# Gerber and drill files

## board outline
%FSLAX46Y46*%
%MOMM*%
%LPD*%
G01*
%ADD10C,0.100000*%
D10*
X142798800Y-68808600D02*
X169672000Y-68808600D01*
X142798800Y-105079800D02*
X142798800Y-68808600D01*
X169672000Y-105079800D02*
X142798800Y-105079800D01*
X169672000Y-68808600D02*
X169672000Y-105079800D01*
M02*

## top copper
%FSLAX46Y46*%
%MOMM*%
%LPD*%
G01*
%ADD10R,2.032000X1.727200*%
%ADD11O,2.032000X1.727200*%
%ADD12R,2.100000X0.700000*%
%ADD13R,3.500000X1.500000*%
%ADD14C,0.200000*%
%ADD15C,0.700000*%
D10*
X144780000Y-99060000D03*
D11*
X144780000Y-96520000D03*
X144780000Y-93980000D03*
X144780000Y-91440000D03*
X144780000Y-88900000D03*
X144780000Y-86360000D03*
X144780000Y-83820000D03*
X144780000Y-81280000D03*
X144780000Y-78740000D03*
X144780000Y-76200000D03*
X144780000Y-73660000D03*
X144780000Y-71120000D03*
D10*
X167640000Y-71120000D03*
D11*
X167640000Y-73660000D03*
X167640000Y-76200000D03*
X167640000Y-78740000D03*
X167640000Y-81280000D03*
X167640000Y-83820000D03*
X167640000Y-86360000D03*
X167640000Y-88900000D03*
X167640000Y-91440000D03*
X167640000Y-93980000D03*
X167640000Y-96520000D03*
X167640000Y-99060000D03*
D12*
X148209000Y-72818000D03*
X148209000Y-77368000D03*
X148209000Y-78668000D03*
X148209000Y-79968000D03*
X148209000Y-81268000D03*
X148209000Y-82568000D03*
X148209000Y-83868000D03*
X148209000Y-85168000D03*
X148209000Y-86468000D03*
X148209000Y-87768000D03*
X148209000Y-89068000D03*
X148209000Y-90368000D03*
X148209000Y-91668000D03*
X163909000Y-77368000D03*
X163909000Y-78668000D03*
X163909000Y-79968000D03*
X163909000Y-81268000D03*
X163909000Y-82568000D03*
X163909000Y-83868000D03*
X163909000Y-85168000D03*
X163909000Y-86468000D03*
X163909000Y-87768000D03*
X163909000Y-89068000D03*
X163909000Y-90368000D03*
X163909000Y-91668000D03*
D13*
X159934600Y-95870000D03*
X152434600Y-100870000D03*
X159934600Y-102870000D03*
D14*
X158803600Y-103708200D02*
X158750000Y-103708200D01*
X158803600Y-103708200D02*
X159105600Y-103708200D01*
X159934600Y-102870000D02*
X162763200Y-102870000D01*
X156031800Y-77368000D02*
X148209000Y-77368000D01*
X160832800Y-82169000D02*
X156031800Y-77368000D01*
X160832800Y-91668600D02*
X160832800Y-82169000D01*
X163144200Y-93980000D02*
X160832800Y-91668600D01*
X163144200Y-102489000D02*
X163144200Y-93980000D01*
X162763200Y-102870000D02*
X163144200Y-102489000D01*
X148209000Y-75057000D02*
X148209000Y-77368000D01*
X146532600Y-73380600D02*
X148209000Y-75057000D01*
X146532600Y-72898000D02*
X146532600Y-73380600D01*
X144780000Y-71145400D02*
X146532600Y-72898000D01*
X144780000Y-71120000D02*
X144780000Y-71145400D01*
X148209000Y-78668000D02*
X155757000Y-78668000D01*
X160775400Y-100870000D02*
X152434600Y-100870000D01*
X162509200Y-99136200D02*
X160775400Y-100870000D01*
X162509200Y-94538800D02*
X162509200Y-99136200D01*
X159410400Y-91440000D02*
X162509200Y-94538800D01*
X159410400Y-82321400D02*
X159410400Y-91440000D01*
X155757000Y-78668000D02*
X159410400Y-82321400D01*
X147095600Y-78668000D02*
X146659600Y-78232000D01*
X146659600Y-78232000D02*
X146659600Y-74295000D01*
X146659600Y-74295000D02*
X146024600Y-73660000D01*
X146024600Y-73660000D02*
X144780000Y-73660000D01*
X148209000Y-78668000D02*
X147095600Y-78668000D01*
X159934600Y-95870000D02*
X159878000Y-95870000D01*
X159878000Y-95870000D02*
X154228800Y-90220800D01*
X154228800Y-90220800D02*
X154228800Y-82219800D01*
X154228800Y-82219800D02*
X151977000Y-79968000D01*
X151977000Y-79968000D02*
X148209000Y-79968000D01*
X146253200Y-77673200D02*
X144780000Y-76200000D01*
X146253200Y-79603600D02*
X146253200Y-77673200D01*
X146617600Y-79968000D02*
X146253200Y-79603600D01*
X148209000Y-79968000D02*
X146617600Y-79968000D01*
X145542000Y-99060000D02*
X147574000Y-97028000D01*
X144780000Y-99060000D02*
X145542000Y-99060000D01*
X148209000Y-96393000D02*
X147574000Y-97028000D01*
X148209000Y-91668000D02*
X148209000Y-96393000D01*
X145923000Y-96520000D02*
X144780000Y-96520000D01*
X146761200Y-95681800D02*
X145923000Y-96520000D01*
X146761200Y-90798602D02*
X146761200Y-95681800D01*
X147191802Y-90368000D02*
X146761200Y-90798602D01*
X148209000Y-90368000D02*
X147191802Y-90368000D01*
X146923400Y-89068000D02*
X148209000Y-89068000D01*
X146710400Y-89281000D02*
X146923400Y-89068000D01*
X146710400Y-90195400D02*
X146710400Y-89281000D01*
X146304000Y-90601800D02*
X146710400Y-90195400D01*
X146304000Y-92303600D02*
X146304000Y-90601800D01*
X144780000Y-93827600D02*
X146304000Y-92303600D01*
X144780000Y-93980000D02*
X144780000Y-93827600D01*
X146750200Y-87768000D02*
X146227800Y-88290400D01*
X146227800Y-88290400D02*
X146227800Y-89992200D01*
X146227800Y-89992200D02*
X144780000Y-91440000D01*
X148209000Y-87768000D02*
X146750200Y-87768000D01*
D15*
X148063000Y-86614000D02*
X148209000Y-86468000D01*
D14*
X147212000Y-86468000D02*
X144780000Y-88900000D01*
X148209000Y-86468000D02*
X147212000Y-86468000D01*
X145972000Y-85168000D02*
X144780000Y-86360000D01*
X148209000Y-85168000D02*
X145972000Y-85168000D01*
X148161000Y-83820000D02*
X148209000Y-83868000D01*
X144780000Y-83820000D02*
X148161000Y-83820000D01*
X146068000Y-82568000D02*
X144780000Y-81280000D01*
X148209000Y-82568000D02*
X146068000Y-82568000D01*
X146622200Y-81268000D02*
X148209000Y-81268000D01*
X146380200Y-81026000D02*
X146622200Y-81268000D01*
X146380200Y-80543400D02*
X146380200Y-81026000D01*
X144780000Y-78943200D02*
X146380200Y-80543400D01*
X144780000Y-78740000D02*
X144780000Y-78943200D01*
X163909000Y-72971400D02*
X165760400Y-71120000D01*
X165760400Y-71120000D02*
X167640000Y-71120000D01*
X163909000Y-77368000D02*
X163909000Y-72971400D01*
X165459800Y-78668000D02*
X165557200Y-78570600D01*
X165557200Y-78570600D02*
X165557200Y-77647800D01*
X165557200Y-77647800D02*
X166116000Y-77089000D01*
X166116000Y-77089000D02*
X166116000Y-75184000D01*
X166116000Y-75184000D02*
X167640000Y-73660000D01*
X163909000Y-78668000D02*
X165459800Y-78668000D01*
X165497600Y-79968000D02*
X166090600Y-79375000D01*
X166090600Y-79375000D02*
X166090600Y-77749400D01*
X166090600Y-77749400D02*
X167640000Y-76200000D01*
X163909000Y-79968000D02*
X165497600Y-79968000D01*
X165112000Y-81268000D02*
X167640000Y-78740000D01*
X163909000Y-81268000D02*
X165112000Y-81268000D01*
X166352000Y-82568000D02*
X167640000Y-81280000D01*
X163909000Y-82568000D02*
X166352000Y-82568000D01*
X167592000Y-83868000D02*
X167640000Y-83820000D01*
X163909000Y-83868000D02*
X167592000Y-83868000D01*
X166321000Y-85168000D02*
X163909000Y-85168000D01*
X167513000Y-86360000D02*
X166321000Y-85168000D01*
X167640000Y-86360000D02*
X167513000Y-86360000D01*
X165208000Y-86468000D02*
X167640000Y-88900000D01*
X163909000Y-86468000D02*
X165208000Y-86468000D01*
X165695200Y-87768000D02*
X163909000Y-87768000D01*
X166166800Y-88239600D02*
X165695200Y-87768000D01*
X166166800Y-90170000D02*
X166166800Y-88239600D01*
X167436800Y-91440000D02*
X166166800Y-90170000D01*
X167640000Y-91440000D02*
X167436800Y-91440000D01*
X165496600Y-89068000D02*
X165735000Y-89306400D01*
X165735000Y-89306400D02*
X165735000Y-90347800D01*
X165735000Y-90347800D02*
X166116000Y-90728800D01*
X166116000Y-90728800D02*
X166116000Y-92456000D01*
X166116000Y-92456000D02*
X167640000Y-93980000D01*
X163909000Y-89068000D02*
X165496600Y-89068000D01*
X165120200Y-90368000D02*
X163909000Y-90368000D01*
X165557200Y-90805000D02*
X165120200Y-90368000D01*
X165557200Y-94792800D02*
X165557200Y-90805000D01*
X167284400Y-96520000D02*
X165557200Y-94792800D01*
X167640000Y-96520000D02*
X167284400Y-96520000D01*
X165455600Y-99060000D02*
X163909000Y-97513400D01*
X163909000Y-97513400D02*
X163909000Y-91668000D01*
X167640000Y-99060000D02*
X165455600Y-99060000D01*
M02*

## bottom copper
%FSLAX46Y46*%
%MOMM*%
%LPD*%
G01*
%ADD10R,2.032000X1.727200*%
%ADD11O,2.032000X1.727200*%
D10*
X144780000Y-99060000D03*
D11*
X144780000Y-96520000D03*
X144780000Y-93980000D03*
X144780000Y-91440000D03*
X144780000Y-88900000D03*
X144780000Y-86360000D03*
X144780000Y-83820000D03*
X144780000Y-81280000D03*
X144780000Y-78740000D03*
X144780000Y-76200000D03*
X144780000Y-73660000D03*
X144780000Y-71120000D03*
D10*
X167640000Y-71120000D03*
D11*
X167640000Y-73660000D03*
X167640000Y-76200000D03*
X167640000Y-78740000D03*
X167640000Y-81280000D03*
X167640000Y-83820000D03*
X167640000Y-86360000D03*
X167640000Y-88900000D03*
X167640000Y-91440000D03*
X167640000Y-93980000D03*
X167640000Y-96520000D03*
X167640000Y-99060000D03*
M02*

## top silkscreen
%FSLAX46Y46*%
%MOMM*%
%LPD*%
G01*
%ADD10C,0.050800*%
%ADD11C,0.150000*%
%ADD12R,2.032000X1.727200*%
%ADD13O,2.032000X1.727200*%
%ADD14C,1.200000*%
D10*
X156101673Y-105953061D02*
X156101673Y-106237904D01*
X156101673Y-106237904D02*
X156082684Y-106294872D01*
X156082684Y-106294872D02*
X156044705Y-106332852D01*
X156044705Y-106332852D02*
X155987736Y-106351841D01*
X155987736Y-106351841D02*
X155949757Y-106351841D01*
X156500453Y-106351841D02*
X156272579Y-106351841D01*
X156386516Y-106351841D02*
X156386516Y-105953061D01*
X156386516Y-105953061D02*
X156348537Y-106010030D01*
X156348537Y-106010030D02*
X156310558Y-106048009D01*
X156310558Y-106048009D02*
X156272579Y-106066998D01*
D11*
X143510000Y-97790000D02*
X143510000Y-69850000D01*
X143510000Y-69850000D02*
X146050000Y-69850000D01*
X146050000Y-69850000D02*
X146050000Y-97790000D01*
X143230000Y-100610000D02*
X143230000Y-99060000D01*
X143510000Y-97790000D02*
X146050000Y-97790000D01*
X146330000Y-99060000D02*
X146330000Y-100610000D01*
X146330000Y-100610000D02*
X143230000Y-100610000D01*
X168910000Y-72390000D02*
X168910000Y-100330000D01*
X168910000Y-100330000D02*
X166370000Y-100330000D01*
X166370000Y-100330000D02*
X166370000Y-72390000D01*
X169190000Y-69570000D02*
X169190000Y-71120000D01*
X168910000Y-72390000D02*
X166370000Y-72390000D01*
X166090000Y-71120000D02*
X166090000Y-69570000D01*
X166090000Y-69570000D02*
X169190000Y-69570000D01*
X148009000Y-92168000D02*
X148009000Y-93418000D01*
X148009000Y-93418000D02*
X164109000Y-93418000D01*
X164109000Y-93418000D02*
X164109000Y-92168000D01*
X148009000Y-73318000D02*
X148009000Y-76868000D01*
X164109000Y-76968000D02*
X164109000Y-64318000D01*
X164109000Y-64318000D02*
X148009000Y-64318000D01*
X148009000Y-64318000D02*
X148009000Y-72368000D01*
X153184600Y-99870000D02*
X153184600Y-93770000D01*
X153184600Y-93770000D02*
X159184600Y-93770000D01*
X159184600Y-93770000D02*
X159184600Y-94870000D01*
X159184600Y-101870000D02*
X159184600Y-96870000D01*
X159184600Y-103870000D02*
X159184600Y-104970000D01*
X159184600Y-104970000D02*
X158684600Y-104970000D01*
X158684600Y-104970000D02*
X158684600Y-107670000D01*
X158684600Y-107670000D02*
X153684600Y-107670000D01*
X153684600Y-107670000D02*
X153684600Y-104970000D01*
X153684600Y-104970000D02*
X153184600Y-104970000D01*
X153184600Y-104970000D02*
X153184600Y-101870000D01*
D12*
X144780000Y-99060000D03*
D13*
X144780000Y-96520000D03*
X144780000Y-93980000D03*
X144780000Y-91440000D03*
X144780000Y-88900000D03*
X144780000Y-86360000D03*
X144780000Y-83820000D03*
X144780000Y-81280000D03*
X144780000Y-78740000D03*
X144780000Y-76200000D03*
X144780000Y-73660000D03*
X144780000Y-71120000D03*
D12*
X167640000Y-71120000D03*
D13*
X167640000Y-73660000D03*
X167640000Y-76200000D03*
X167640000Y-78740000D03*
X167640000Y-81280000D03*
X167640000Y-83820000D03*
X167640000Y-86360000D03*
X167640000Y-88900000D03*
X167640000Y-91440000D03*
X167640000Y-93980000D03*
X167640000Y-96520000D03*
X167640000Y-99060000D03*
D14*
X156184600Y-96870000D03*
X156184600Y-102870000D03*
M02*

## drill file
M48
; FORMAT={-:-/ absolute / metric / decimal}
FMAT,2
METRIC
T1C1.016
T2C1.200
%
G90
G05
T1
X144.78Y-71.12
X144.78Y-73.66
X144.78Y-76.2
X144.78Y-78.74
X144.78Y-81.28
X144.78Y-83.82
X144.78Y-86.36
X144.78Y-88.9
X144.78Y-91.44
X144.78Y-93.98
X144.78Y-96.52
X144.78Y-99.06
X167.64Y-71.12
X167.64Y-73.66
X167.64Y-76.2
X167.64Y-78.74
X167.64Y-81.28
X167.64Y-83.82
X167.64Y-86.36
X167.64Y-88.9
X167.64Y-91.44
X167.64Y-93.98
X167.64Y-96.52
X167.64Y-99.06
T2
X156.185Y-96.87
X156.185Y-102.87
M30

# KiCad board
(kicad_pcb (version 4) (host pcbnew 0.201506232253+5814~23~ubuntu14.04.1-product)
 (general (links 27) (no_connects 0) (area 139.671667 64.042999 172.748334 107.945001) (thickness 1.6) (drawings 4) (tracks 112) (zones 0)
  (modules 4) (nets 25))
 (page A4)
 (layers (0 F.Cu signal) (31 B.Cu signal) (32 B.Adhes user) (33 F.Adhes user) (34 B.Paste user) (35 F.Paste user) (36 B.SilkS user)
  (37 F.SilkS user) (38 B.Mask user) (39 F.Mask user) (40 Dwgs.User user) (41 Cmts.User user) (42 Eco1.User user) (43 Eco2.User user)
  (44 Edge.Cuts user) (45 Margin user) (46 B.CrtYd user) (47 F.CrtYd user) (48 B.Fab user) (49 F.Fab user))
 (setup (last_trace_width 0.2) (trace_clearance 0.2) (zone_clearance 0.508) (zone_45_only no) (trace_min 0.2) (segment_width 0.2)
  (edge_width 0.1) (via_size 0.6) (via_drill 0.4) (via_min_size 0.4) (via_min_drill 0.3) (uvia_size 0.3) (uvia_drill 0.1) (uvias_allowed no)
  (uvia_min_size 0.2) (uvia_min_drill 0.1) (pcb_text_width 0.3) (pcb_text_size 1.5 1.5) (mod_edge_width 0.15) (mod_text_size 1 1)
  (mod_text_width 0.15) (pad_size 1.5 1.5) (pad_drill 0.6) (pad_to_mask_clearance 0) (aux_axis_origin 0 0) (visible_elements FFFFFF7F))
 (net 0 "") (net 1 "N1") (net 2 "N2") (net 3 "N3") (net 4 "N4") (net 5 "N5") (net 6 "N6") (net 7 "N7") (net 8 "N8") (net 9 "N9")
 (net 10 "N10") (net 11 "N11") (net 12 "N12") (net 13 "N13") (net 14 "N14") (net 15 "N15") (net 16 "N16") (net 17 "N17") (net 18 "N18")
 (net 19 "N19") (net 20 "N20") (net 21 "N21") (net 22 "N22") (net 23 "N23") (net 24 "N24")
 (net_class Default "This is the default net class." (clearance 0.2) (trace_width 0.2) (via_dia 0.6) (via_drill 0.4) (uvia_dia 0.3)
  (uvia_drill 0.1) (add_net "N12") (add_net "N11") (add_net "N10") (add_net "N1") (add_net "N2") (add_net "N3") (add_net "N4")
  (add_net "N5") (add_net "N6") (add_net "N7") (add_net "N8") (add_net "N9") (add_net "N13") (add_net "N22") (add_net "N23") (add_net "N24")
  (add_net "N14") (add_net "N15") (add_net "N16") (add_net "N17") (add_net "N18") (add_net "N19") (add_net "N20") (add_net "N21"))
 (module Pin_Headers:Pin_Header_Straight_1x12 (layer F.Cu) (at 144.78 99.06 180)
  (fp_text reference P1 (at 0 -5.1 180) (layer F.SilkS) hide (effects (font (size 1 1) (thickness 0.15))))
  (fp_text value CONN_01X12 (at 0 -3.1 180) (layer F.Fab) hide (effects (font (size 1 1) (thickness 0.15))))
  (fp_line (start 1.27 1.27) (end 1.27 29.21) (layer F.SilkS) (width 0.15))
  (fp_line (start 1.27 29.21) (end -1.27 29.21) (layer F.SilkS) (width 0.15))
  (fp_line (start -1.27 29.21) (end -1.27 1.27) (layer F.SilkS) (width 0.15))
  (fp_line (start 1.55 -1.55) (end 1.55 0) (layer F.SilkS) (width 0.15))
  (fp_line (start 1.27 1.27) (end -1.27 1.27) (layer F.SilkS) (width 0.15))
  (fp_line (start -1.55 0) (end -1.55 -1.55) (layer F.SilkS) (width 0.15))
  (fp_line (start -1.55 -1.55) (end 1.55 -1.55) (layer F.SilkS) (width 0.15))
  (pad 1 thru_hole rect (at 0 0 180) (size 2.032 1.7272) (drill 1.016) (layers *.Cu *.Mask F.SilkS) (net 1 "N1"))
  (pad 2 thru_hole oval (at 0 2.54 180) (size 2.032 1.7272) (drill 1.016) (layers *.Cu *.Mask F.SilkS) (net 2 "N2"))
  (pad 3 thru_hole oval (at 0 5.08 180) (size 2.032 1.7272) (drill 1.016) (layers *.Cu *.Mask F.SilkS) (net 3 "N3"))
  (pad 4 thru_hole oval (at 0 7.62 180) (size 2.032 1.7272) (drill 1.016) (layers *.Cu *.Mask F.SilkS) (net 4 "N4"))
  (pad 5 thru_hole oval (at 0 10.16 180) (size 2.032 1.7272) (drill 1.016) (layers *.Cu *.Mask F.SilkS) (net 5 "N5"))
  (pad 6 thru_hole oval (at 0 12.7 180) (size 2.032 1.7272) (drill 1.016) (layers *.Cu *.Mask F.SilkS) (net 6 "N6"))
  (pad 7 thru_hole oval (at 0 15.24 180) (size 2.032 1.7272) (drill 1.016) (layers *.Cu *.Mask F.SilkS) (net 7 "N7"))
  (pad 8 thru_hole oval (at 0 17.78 180) (size 2.032 1.7272) (drill 1.016) (layers *.Cu *.Mask F.SilkS) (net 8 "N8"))
  (pad 9 thru_hole oval (at 0 20.32 180) (size 2.032 1.7272) (drill 1.016) (layers *.Cu *.Mask F.SilkS) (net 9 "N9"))
  (pad 10 thru_hole oval (at 0 22.86 180) (size 2.032 1.7272) (drill 1.016) (layers *.Cu *.Mask F.SilkS) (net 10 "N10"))
  (pad 11 thru_hole oval (at 0 25.4 180) (size 2.032 1.7272) (drill 1.016) (layers *.Cu *.Mask F.SilkS) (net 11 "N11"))
  (pad 12 thru_hole oval (at 0 27.94 180) (size 2.032 1.7272) (drill 1.016) (layers *.Cu *.Mask F.SilkS) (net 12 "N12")))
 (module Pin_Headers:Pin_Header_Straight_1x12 (layer F.Cu) (at 167.64 71.12)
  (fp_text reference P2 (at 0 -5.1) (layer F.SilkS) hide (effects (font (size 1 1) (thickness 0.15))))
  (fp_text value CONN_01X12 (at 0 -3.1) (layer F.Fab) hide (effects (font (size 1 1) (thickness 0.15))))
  (fp_line (start 1.27 1.27) (end 1.27 29.21) (layer F.SilkS) (width 0.15))
  (fp_line (start 1.27 29.21) (end -1.27 29.21) (layer F.SilkS) (width 0.15))
  (fp_line (start -1.27 29.21) (end -1.27 1.27) (layer F.SilkS) (width 0.15))
  (fp_line (start 1.55 -1.55) (end 1.55 0) (layer F.SilkS) (width 0.15))
  (fp_line (start 1.27 1.27) (end -1.27 1.27) (layer F.SilkS) (width 0.15))
  (fp_line (start -1.55 0) (end -1.55 -1.55) (layer F.SilkS) (width 0.15))
  (fp_line (start -1.55 -1.55) (end 1.55 -1.55) (layer F.SilkS) (width 0.15))
  (pad 1 thru_hole rect (at 0 0) (size 2.032 1.7272) (drill 1.016) (layers *.Cu *.Mask F.SilkS) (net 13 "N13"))
  (pad 2 thru_hole oval (at 0 2.54) (size 2.032 1.7272) (drill 1.016) (layers *.Cu *.Mask F.SilkS) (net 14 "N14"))
  (pad 3 thru_hole oval (at 0 5.08) (size 2.032 1.7272) (drill 1.016) (layers *.Cu *.Mask F.SilkS) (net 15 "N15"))
  (pad 4 thru_hole oval (at 0 7.62) (size 2.032 1.7272) (drill 1.016) (layers *.Cu *.Mask F.SilkS) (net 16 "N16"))
  (pad 5 thru_hole oval (at 0 10.16) (size 2.032 1.7272) (drill 1.016) (layers *.Cu *.Mask F.SilkS) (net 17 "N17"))
  (pad 6 thru_hole oval (at 0 12.7) (size 2.032 1.7272) (drill 1.016) (layers *.Cu *.Mask F.SilkS) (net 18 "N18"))
  (pad 7 thru_hole oval (at 0 15.24) (size 2.032 1.7272) (drill 1.016) (layers *.Cu *.Mask F.SilkS) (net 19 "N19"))
  (pad 8 thru_hole oval (at 0 17.78) (size 2.032 1.7272) (drill 1.016) (layers *.Cu *.Mask F.SilkS) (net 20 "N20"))
  (pad 9 thru_hole oval (at 0 20.32) (size 2.032 1.7272) (drill 1.016) (layers *.Cu *.Mask F.SilkS) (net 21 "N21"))
  (pad 10 thru_hole oval (at 0 22.86) (size 2.032 1.7272) (drill 1.016) (layers *.Cu *.Mask F.SilkS) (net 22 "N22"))
  (pad 11 thru_hole oval (at 0 25.4) (size 2.032 1.7272) (drill 1.016) (layers *.Cu *.Mask F.SilkS) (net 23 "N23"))
  (pad 12 thru_hole oval (at 0 27.94) (size 2.032 1.7272) (drill 1.016) (layers *.Cu *.Mask F.SilkS) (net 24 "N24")))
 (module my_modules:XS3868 (layer F.Cu) (at 148.209 93.218)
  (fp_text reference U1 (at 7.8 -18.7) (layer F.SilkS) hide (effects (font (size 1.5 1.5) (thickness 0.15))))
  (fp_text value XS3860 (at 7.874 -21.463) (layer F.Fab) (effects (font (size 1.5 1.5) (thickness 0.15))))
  (fp_line (start -0.2 -1.05) (end -0.2 0.2) (layer F.SilkS) (width 0.15))
  (fp_line (start -0.2 0.2) (end 15.9 0.2) (layer F.SilkS) (width 0.15))
  (fp_line (start 15.9 0.2) (end 15.9 -1.05) (layer F.SilkS) (width 0.15))
  (fp_line (start -0.2 -19.9) (end -0.2 -16.35) (layer F.SilkS) (width 0.15))
  (fp_line (start 15.9 -16.25) (end 15.9 -28.9) (layer F.SilkS) (width 0.15))
  (fp_line (start 15.9 -28.9) (end -0.2 -28.9) (layer F.SilkS) (width 0.15))
  (fp_line (start -0.2 -28.9) (end -0.2 -20.85) (layer F.SilkS) (width 0.15))
  (pad 1 smd rect (at 0 -20.4) (size 2.1 0.7) (layers F.Cu F.Paste F.Mask))
  (pad 2 smd rect (at 0 -15.85) (size 2.1 0.7) (layers F.Cu F.Paste F.Mask) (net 12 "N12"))
  (pad 3 smd rect (at 0 -14.55) (size 2.1 0.7) (layers F.Cu F.Paste F.Mask) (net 11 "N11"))
  (pad 4 smd rect (at 0 -13.25) (size 2.1 0.7) (layers F.Cu F.Paste F.Mask) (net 10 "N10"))
  (pad 5 smd rect (at 0 -11.95) (size 2.1 0.7) (layers F.Cu F.Paste F.Mask) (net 9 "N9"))
  (pad 6 smd rect (at 0 -10.65) (size 2.1 0.7) (layers F.Cu F.Paste F.Mask) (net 8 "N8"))
  (pad 7 smd rect (at 0 -9.35) (size 2.1 0.7) (layers F.Cu F.Paste F.Mask) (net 7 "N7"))
  (pad 8 smd rect (at 0 -8.05) (size 2.1 0.7) (layers F.Cu F.Paste F.Mask) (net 6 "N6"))
  (pad 9 smd rect (at 0 -6.75) (size 2.1 0.7) (layers F.Cu F.Paste F.Mask) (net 5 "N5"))
  (pad 10 smd rect (at 0 -5.45) (size 2.1 0.7) (layers F.Cu F.Paste F.Mask) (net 4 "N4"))
  (pad 11 smd rect (at 0 -4.15) (size 2.1 0.7) (layers F.Cu F.Paste F.Mask) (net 3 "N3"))
  (pad 12 smd rect (at 0 -2.85) (size 2.1 0.7) (layers F.Cu F.Paste F.Mask) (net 2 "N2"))
  (pad 13 smd rect (at 0 -1.55) (size 2.1 0.7) (layers F.Cu F.Paste F.Mask) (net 1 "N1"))
  (pad 25 smd rect (at 15.7 -15.85) (size 2.1 0.7) (layers F.Cu F.Paste F.Mask) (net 13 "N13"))
  (pad 24 smd rect (at 15.7 -14.55) (size 2.1 0.7) (layers F.Cu F.Paste F.Mask) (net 14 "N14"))
  (pad 23 smd rect (at 15.7 -13.25) (size 2.1 0.7) (layers F.Cu F.Paste F.Mask) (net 15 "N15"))
  (pad 22 smd rect (at 15.7 -11.95) (size 2.1 0.7) (layers F.Cu F.Paste F.Mask) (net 16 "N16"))
  (pad 21 smd rect (at 15.7 -10.65) (size 2.1 0.7) (layers F.Cu F.Paste F.Mask) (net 17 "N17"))
  (pad 20 smd rect (at 15.7 -9.35) (size 2.1 0.7) (layers F.Cu F.Paste F.Mask) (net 18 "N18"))
  (pad 19 smd rect (at 15.7 -8.05) (size 2.1 0.7) (layers F.Cu F.Paste F.Mask) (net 19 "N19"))
  (pad 18 smd rect (at 15.7 -6.75) (size 2.1 0.7) (layers F.Cu F.Paste F.Mask) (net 20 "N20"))
  (pad 17 smd rect (at 15.7 -5.45) (size 2.1 0.7) (layers F.Cu F.Paste F.Mask) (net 21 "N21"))
  (pad 16 smd rect (at 15.7 -4.15) (size 2.1 0.7) (layers F.Cu F.Paste F.Mask) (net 22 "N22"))
  (pad 15 smd rect (at 15.7 -2.85) (size 2.1 0.7) (layers F.Cu F.Paste F.Mask) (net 23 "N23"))
  (pad 14 smd rect (at 15.7 -1.55) (size 2.1 0.7) (layers F.Cu F.Paste F.Mask) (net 24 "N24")))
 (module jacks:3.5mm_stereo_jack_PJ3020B (layer F.Cu) (at 156.1846 102.87 180)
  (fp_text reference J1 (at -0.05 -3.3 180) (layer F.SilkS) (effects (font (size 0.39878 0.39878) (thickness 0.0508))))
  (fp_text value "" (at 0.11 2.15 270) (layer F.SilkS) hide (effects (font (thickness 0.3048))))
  (fp_line (start 3 3) (end 3 9.1) (layer F.SilkS) (width 0.15))
  (fp_line (start 3 9.1) (end -3 9.1) (layer F.SilkS) (width 0.15))
  (fp_line (start -3 9.1) (end -3 8) (layer F.SilkS) (width 0.15))
  (fp_line (start -3 1) (end -3 6) (layer F.SilkS) (width 0.15))
  (fp_line (start -3 -1) (end -3 -2.1) (layer F.SilkS) (width 0.15))
  (fp_line (start -3 -2.1) (end -2.5 -2.1) (layer F.SilkS) (width 0.15))
  (fp_line (start -2.5 -2.1) (end -2.5 -4.8) (layer F.SilkS) (width 0.15))
  (fp_line (start -2.5 -4.8) (end 2.5 -4.8) (layer F.SilkS) (width 0.15))
  (fp_line (start 2.5 -4.8) (end 2.5 -2.1) (layer F.SilkS) (width 0.15))
  (fp_line (start 2.5 -2.1) (end 3 -2.1) (layer F.SilkS) (width 0.15))
  (fp_line (start 3 -2.1) (end 3 1) (layer F.SilkS) (width 0.15))
  (pad "" np_thru_hole circle (at 0 6 180) (size 1.2 1.2) (drill 1.2) (layers *.Cu *.Mask F.SilkS))
  (pad 5 smd rect (at -3.75 7 180) (size 3.5 1.5) (layers F.Cu F.Paste F.Mask) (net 10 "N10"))
  (pad 2 smd rect (at 3.75 2 180) (size 3.5 1.5) (layers F.Cu F.Paste F.Mask) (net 11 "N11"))
  (pad 1 smd rect (at -3.75 0 180) (size 3.5 1.5) (layers F.Cu F.Paste F.Mask) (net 12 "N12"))
  (pad "" np_thru_hole circle (at 0 0 180) (size 1.2 1.2) (drill 1.2) (layers *.Cu *.Mask F.SilkS)))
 (gr_line (start 142.7988 68.8086) (end 169.672 68.8086) (angle 90) (layer Edge.Cuts) (width 0.1))
 (gr_line (start 142.7988 105.0798) (end 142.7988 68.8086) (angle 90) (layer Edge.Cuts) (width 0.1))
 (gr_line (start 169.672 105.0798) (end 142.7988 105.0798) (angle 90) (layer Edge.Cuts) (width 0.1))
 (gr_line (start 169.672 68.8086) (end 169.672 105.0798) (angle 90) (layer Edge.Cuts) (width 0.1))
 (segment (start 158.8036 103.7082) (end 158.75 103.7082) (width 0.2) (layer F.Cu) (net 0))
 (segment (start 158.8036 103.7082) (end 159.1056 103.7082) (width 0.2) (layer F.Cu) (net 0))
 (segment (start 159.9346 102.87) (end 162.7632 102.87) (width 0.2) (layer F.Cu) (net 12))
 (segment (start 156.0318 77.368) (end 148.209 77.368) (width 0.2) (layer F.Cu) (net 12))
 (segment (start 160.8328 82.169) (end 156.0318 77.368) (width 0.2) (layer F.Cu) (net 12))
 (segment (start 160.8328 91.6686) (end 160.8328 82.169) (width 0.2) (layer F.Cu) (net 12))
 (segment (start 163.1442 93.98) (end 160.8328 91.6686) (width 0.2) (layer F.Cu) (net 12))
 (segment (start 163.1442 102.489) (end 163.1442 93.98) (width 0.2) (layer F.Cu) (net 12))
 (segment (start 162.7632 102.87) (end 163.1442 102.489) (width 0.2) (layer F.Cu) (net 12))
 (segment (start 148.209 75.057) (end 148.209 77.368) (width 0.2) (layer F.Cu) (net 12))
 (segment (start 146.5326 73.3806) (end 148.209 75.057) (width 0.2) (layer F.Cu) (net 12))
 (segment (start 146.5326 72.898) (end 146.5326 73.3806) (width 0.2) (layer F.Cu) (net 12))
 (segment (start 144.78 71.1454) (end 146.5326 72.898) (width 0.2) (layer F.Cu) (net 12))
 (segment (start 144.78 71.12) (end 144.78 71.1454) (width 0.2) (layer F.Cu) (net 12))
 (segment (start 148.209 78.668) (end 155.757 78.668) (width 0.2) (layer F.Cu) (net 11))
 (segment (start 160.7754 100.87) (end 152.4346 100.87) (width 0.2) (layer F.Cu) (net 11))
 (segment (start 162.5092 99.1362) (end 160.7754 100.87) (width 0.2) (layer F.Cu) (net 11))
 (segment (start 162.5092 94.5388) (end 162.5092 99.1362) (width 0.2) (layer F.Cu) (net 11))
 (segment (start 159.4104 91.44) (end 162.5092 94.5388) (width 0.2) (layer F.Cu) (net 11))
 (segment (start 159.4104 82.3214) (end 159.4104 91.44) (width 0.2) (layer F.Cu) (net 11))
 (segment (start 155.757 78.668) (end 159.4104 82.3214) (width 0.2) (layer F.Cu) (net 11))
 (segment (start 147.0956 78.668) (end 146.6596 78.232) (width 0.2) (layer F.Cu) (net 11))
 (segment (start 146.6596 78.232) (end 146.6596 74.295) (width 0.2) (layer F.Cu) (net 11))
 (segment (start 146.6596 74.295) (end 146.0246 73.66) (width 0.2) (layer F.Cu) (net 11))
 (segment (start 146.0246 73.66) (end 144.78 73.66) (width 0.2) (layer F.Cu) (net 11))
 (segment (start 148.209 78.668) (end 147.0956 78.668) (width 0.2) (layer F.Cu) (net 11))
 (segment (start 159.9346 95.87) (end 159.878 95.87) (width 0.2) (layer F.Cu) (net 10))
 (segment (start 159.878 95.87) (end 154.2288 90.2208) (width 0.2) (layer F.Cu) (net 10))
 (segment (start 154.2288 90.2208) (end 154.2288 82.2198) (width 0.2) (layer F.Cu) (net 10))
 (segment (start 154.2288 82.2198) (end 151.977 79.968) (width 0.2) (layer F.Cu) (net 10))
 (segment (start 151.977 79.968) (end 148.209 79.968) (width 0.2) (layer F.Cu) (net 10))
 (segment (start 146.2532 77.6732) (end 144.78 76.2) (width 0.2) (layer F.Cu) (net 10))
 (segment (start 146.2532 79.6036) (end 146.2532 77.6732) (width 0.2) (layer F.Cu) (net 10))
 (segment (start 146.6176 79.968) (end 146.2532 79.6036) (width 0.2) (layer F.Cu) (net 10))
 (segment (start 148.209 79.968) (end 146.6176 79.968) (width 0.2) (layer F.Cu) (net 10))
 (segment (start 145.542 99.06) (end 147.574 97.028) (width 0.2) (layer F.Cu) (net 1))
 (segment (start 144.78 99.06) (end 145.542 99.06) (width 0.2) (layer F.Cu) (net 1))
 (segment (start 148.209 96.393) (end 147.574 97.028) (width 0.2) (layer F.Cu) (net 1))
 (segment (start 148.209 91.668) (end 148.209 96.393) (width 0.2) (layer F.Cu) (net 1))
 (segment (start 145.923 96.52) (end 144.78 96.52) (width 0.2) (layer F.Cu) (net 2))
 (segment (start 146.7612 95.6818) (end 145.923 96.52) (width 0.2) (layer F.Cu) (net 2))
 (segment (start 146.7612 90.798602) (end 146.7612 95.6818) (width 0.2) (layer F.Cu) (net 2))
 (segment (start 147.191802 90.368) (end 146.7612 90.798602) (width 0.2) (layer F.Cu) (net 2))
 (segment (start 148.209 90.368) (end 147.191802 90.368) (width 0.2) (layer F.Cu) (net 2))
 (segment (start 146.9234 89.068) (end 148.209 89.068) (width 0.2) (layer F.Cu) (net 3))
 (segment (start 146.7104 89.281) (end 146.9234 89.068) (width 0.2) (layer F.Cu) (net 3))
 (segment (start 146.7104 90.1954) (end 146.7104 89.281) (width 0.2) (layer F.Cu) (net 3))
 (segment (start 146.304 90.6018) (end 146.7104 90.1954) (width 0.2) (layer F.Cu) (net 3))
 (segment (start 146.304 92.3036) (end 146.304 90.6018) (width 0.2) (layer F.Cu) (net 3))
 (segment (start 144.78 93.8276) (end 146.304 92.3036) (width 0.2) (layer F.Cu) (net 3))
 (segment (start 144.78 93.98) (end 144.78 93.8276) (width 0.2) (layer F.Cu) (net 3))
 (segment (start 146.7502 87.768) (end 146.2278 88.2904) (width 0.2) (layer F.Cu) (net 4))
 (segment (start 146.2278 88.2904) (end 146.2278 89.9922) (width 0.2) (layer F.Cu) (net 4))
 (segment (start 146.2278 89.9922) (end 144.78 91.44) (width 0.2) (layer F.Cu) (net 4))
 (segment (start 148.209 87.768) (end 146.7502 87.768) (width 0.2) (layer F.Cu) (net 4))
 (segment (start 148.063 86.614) (end 148.209 86.468) (width 0.7) (layer F.Cu) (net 5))
 (segment (start 147.212 86.468) (end 144.78 88.9) (width 0.2) (layer F.Cu) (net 5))
 (segment (start 148.209 86.468) (end 147.212 86.468) (width 0.2) (layer F.Cu) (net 5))
 (segment (start 145.972 85.168) (end 144.78 86.36) (width 0.2) (layer F.Cu) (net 6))
 (segment (start 148.209 85.168) (end 145.972 85.168) (width 0.2) (layer F.Cu) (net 6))
 (segment (start 148.161 83.82) (end 148.209 83.868) (width 0.2) (layer F.Cu) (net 7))
 (segment (start 144.78 83.82) (end 148.161 83.82) (width 0.2) (layer F.Cu) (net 7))
 (segment (start 146.068 82.568) (end 144.78 81.28) (width 0.2) (layer F.Cu) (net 8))
 (segment (start 148.209 82.568) (end 146.068 82.568) (width 0.2) (layer F.Cu) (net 8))
 (segment (start 146.6222 81.268) (end 148.209 81.268) (width 0.2) (layer F.Cu) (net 9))
 (segment (start 146.3802 81.026) (end 146.6222 81.268) (width 0.2) (layer F.Cu) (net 9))
 (segment (start 146.3802 80.5434) (end 146.3802 81.026) (width 0.2) (layer F.Cu) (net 9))
 (segment (start 144.78 78.9432) (end 146.3802 80.5434) (width 0.2) (layer F.Cu) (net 9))
 (segment (start 144.78 78.74) (end 144.78 78.9432) (width 0.2) (layer F.Cu) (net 9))
 (segment (start 163.909 72.9714) (end 165.7604 71.12) (width 0.2) (layer F.Cu) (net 13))
 (segment (start 165.7604 71.12) (end 167.64 71.12) (width 0.2) (layer F.Cu) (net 13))
 (segment (start 163.909 77.368) (end 163.909 72.9714) (width 0.2) (layer F.Cu) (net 13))
 (segment (start 165.4598 78.668) (end 165.5572 78.5706) (width 0.2) (layer F.Cu) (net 14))
 (segment (start 165.5572 78.5706) (end 165.5572 77.6478) (width 0.2) (layer F.Cu) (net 14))
 (segment (start 165.5572 77.6478) (end 166.116 77.089) (width 0.2) (layer F.Cu) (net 14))
 (segment (start 166.116 77.089) (end 166.116 75.184) (width 0.2) (layer F.Cu) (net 14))
 (segment (start 166.116 75.184) (end 167.64 73.66) (width 0.2) (layer F.Cu) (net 14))
 (segment (start 163.909 78.668) (end 165.4598 78.668) (width 0.2) (layer F.Cu) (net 14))
 (segment (start 165.4976 79.968) (end 166.0906 79.375) (width 0.2) (layer F.Cu) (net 15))
 (segment (start 166.0906 79.375) (end 166.0906 77.7494) (width 0.2) (layer F.Cu) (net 15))
 (segment (start 166.0906 77.7494) (end 167.64 76.2) (width 0.2) (layer F.Cu) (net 15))
 (segment (start 163.909 79.968) (end 165.4976 79.968) (width 0.2) (layer F.Cu) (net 15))
 (segment (start 165.112 81.268) (end 167.64 78.74) (width 0.2) (layer F.Cu) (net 16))
 (segment (start 163.909 81.268) (end 165.112 81.268) (width 0.2) (layer F.Cu) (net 16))
 (segment (start 166.352 82.568) (end 167.64 81.28) (width 0.2) (layer F.Cu) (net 17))
 (segment (start 163.909 82.568) (end 166.352 82.568) (width 0.2) (layer F.Cu) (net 17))
 (segment (start 167.592 83.868) (end 167.64 83.82) (width 0.2) (layer F.Cu) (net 18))
 (segment (start 163.909 83.868) (end 167.592 83.868) (width 0.2) (layer F.Cu) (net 18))
 (segment (start 166.321 85.168) (end 163.909 85.168) (width 0.2) (layer F.Cu) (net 19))
 (segment (start 167.513 86.36) (end 166.321 85.168) (width 0.2) (layer F.Cu) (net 19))
 (segment (start 167.64 86.36) (end 167.513 86.36) (width 0.2) (layer F.Cu) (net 19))
 (segment (start 165.208 86.468) (end 167.64 88.9) (width 0.2) (layer F.Cu) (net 20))
 (segment (start 163.909 86.468) (end 165.208 86.468) (width 0.2) (layer F.Cu) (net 20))
 (segment (start 165.6952 87.768) (end 163.909 87.768) (width 0.2) (layer F.Cu) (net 21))
 (segment (start 166.1668 88.2396) (end 165.6952 87.768) (width 0.2) (layer F.Cu) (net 21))
 (segment (start 166.1668 90.17) (end 166.1668 88.2396) (width 0.2) (layer F.Cu) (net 21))
 (segment (start 167.4368 91.44) (end 166.1668 90.17) (width 0.2) (layer F.Cu) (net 21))
 (segment (start 167.64 91.44) (end 167.4368 91.44) (width 0.2) (layer F.Cu) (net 21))
 (segment (start 165.4966 89.068) (end 165.735 89.3064) (width 0.2) (layer F.Cu) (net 22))
 (segment (start 165.735 89.3064) (end 165.735 90.3478) (width 0.2) (layer F.Cu) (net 22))
 (segment (start 165.735 90.3478) (end 166.116 90.7288) (width 0.2) (layer F.Cu) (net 22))
 (segment (start 166.116 90.7288) (end 166.116 92.456) (width 0.2) (layer F.Cu) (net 22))
 (segment (start 166.116 92.456) (end 167.64 93.98) (width 0.2) (layer F.Cu) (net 22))
 (segment (start 163.909 89.068) (end 165.4966 89.068) (width 0.2) (layer F.Cu) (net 22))
 (segment (start 165.1202 90.368) (end 163.909 90.368) (width 0.2) (layer F.Cu) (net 23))
 (segment (start 165.5572 90.805) (end 165.1202 90.368) (width 0.2) (layer F.Cu) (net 23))
 (segment (start 165.5572 94.7928) (end 165.5572 90.805) (width 0.2) (layer F.Cu) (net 23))
 (segment (start 167.2844 96.52) (end 165.5572 94.7928) (width 0.2) (layer F.Cu) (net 23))
 (segment (start 167.64 96.52) (end 167.2844 96.52) (width 0.2) (layer F.Cu) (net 23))
 (segment (start 165.4556 99.06) (end 163.909 97.5134) (width 0.2) (layer F.Cu) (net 24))
 (segment (start 163.909 97.5134) (end 163.909 91.668) (width 0.2) (layer F.Cu) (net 24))
 (segment (start 167.64 99.06) (end 165.4556 99.06) (width 0.2) (layer F.Cu) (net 24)))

